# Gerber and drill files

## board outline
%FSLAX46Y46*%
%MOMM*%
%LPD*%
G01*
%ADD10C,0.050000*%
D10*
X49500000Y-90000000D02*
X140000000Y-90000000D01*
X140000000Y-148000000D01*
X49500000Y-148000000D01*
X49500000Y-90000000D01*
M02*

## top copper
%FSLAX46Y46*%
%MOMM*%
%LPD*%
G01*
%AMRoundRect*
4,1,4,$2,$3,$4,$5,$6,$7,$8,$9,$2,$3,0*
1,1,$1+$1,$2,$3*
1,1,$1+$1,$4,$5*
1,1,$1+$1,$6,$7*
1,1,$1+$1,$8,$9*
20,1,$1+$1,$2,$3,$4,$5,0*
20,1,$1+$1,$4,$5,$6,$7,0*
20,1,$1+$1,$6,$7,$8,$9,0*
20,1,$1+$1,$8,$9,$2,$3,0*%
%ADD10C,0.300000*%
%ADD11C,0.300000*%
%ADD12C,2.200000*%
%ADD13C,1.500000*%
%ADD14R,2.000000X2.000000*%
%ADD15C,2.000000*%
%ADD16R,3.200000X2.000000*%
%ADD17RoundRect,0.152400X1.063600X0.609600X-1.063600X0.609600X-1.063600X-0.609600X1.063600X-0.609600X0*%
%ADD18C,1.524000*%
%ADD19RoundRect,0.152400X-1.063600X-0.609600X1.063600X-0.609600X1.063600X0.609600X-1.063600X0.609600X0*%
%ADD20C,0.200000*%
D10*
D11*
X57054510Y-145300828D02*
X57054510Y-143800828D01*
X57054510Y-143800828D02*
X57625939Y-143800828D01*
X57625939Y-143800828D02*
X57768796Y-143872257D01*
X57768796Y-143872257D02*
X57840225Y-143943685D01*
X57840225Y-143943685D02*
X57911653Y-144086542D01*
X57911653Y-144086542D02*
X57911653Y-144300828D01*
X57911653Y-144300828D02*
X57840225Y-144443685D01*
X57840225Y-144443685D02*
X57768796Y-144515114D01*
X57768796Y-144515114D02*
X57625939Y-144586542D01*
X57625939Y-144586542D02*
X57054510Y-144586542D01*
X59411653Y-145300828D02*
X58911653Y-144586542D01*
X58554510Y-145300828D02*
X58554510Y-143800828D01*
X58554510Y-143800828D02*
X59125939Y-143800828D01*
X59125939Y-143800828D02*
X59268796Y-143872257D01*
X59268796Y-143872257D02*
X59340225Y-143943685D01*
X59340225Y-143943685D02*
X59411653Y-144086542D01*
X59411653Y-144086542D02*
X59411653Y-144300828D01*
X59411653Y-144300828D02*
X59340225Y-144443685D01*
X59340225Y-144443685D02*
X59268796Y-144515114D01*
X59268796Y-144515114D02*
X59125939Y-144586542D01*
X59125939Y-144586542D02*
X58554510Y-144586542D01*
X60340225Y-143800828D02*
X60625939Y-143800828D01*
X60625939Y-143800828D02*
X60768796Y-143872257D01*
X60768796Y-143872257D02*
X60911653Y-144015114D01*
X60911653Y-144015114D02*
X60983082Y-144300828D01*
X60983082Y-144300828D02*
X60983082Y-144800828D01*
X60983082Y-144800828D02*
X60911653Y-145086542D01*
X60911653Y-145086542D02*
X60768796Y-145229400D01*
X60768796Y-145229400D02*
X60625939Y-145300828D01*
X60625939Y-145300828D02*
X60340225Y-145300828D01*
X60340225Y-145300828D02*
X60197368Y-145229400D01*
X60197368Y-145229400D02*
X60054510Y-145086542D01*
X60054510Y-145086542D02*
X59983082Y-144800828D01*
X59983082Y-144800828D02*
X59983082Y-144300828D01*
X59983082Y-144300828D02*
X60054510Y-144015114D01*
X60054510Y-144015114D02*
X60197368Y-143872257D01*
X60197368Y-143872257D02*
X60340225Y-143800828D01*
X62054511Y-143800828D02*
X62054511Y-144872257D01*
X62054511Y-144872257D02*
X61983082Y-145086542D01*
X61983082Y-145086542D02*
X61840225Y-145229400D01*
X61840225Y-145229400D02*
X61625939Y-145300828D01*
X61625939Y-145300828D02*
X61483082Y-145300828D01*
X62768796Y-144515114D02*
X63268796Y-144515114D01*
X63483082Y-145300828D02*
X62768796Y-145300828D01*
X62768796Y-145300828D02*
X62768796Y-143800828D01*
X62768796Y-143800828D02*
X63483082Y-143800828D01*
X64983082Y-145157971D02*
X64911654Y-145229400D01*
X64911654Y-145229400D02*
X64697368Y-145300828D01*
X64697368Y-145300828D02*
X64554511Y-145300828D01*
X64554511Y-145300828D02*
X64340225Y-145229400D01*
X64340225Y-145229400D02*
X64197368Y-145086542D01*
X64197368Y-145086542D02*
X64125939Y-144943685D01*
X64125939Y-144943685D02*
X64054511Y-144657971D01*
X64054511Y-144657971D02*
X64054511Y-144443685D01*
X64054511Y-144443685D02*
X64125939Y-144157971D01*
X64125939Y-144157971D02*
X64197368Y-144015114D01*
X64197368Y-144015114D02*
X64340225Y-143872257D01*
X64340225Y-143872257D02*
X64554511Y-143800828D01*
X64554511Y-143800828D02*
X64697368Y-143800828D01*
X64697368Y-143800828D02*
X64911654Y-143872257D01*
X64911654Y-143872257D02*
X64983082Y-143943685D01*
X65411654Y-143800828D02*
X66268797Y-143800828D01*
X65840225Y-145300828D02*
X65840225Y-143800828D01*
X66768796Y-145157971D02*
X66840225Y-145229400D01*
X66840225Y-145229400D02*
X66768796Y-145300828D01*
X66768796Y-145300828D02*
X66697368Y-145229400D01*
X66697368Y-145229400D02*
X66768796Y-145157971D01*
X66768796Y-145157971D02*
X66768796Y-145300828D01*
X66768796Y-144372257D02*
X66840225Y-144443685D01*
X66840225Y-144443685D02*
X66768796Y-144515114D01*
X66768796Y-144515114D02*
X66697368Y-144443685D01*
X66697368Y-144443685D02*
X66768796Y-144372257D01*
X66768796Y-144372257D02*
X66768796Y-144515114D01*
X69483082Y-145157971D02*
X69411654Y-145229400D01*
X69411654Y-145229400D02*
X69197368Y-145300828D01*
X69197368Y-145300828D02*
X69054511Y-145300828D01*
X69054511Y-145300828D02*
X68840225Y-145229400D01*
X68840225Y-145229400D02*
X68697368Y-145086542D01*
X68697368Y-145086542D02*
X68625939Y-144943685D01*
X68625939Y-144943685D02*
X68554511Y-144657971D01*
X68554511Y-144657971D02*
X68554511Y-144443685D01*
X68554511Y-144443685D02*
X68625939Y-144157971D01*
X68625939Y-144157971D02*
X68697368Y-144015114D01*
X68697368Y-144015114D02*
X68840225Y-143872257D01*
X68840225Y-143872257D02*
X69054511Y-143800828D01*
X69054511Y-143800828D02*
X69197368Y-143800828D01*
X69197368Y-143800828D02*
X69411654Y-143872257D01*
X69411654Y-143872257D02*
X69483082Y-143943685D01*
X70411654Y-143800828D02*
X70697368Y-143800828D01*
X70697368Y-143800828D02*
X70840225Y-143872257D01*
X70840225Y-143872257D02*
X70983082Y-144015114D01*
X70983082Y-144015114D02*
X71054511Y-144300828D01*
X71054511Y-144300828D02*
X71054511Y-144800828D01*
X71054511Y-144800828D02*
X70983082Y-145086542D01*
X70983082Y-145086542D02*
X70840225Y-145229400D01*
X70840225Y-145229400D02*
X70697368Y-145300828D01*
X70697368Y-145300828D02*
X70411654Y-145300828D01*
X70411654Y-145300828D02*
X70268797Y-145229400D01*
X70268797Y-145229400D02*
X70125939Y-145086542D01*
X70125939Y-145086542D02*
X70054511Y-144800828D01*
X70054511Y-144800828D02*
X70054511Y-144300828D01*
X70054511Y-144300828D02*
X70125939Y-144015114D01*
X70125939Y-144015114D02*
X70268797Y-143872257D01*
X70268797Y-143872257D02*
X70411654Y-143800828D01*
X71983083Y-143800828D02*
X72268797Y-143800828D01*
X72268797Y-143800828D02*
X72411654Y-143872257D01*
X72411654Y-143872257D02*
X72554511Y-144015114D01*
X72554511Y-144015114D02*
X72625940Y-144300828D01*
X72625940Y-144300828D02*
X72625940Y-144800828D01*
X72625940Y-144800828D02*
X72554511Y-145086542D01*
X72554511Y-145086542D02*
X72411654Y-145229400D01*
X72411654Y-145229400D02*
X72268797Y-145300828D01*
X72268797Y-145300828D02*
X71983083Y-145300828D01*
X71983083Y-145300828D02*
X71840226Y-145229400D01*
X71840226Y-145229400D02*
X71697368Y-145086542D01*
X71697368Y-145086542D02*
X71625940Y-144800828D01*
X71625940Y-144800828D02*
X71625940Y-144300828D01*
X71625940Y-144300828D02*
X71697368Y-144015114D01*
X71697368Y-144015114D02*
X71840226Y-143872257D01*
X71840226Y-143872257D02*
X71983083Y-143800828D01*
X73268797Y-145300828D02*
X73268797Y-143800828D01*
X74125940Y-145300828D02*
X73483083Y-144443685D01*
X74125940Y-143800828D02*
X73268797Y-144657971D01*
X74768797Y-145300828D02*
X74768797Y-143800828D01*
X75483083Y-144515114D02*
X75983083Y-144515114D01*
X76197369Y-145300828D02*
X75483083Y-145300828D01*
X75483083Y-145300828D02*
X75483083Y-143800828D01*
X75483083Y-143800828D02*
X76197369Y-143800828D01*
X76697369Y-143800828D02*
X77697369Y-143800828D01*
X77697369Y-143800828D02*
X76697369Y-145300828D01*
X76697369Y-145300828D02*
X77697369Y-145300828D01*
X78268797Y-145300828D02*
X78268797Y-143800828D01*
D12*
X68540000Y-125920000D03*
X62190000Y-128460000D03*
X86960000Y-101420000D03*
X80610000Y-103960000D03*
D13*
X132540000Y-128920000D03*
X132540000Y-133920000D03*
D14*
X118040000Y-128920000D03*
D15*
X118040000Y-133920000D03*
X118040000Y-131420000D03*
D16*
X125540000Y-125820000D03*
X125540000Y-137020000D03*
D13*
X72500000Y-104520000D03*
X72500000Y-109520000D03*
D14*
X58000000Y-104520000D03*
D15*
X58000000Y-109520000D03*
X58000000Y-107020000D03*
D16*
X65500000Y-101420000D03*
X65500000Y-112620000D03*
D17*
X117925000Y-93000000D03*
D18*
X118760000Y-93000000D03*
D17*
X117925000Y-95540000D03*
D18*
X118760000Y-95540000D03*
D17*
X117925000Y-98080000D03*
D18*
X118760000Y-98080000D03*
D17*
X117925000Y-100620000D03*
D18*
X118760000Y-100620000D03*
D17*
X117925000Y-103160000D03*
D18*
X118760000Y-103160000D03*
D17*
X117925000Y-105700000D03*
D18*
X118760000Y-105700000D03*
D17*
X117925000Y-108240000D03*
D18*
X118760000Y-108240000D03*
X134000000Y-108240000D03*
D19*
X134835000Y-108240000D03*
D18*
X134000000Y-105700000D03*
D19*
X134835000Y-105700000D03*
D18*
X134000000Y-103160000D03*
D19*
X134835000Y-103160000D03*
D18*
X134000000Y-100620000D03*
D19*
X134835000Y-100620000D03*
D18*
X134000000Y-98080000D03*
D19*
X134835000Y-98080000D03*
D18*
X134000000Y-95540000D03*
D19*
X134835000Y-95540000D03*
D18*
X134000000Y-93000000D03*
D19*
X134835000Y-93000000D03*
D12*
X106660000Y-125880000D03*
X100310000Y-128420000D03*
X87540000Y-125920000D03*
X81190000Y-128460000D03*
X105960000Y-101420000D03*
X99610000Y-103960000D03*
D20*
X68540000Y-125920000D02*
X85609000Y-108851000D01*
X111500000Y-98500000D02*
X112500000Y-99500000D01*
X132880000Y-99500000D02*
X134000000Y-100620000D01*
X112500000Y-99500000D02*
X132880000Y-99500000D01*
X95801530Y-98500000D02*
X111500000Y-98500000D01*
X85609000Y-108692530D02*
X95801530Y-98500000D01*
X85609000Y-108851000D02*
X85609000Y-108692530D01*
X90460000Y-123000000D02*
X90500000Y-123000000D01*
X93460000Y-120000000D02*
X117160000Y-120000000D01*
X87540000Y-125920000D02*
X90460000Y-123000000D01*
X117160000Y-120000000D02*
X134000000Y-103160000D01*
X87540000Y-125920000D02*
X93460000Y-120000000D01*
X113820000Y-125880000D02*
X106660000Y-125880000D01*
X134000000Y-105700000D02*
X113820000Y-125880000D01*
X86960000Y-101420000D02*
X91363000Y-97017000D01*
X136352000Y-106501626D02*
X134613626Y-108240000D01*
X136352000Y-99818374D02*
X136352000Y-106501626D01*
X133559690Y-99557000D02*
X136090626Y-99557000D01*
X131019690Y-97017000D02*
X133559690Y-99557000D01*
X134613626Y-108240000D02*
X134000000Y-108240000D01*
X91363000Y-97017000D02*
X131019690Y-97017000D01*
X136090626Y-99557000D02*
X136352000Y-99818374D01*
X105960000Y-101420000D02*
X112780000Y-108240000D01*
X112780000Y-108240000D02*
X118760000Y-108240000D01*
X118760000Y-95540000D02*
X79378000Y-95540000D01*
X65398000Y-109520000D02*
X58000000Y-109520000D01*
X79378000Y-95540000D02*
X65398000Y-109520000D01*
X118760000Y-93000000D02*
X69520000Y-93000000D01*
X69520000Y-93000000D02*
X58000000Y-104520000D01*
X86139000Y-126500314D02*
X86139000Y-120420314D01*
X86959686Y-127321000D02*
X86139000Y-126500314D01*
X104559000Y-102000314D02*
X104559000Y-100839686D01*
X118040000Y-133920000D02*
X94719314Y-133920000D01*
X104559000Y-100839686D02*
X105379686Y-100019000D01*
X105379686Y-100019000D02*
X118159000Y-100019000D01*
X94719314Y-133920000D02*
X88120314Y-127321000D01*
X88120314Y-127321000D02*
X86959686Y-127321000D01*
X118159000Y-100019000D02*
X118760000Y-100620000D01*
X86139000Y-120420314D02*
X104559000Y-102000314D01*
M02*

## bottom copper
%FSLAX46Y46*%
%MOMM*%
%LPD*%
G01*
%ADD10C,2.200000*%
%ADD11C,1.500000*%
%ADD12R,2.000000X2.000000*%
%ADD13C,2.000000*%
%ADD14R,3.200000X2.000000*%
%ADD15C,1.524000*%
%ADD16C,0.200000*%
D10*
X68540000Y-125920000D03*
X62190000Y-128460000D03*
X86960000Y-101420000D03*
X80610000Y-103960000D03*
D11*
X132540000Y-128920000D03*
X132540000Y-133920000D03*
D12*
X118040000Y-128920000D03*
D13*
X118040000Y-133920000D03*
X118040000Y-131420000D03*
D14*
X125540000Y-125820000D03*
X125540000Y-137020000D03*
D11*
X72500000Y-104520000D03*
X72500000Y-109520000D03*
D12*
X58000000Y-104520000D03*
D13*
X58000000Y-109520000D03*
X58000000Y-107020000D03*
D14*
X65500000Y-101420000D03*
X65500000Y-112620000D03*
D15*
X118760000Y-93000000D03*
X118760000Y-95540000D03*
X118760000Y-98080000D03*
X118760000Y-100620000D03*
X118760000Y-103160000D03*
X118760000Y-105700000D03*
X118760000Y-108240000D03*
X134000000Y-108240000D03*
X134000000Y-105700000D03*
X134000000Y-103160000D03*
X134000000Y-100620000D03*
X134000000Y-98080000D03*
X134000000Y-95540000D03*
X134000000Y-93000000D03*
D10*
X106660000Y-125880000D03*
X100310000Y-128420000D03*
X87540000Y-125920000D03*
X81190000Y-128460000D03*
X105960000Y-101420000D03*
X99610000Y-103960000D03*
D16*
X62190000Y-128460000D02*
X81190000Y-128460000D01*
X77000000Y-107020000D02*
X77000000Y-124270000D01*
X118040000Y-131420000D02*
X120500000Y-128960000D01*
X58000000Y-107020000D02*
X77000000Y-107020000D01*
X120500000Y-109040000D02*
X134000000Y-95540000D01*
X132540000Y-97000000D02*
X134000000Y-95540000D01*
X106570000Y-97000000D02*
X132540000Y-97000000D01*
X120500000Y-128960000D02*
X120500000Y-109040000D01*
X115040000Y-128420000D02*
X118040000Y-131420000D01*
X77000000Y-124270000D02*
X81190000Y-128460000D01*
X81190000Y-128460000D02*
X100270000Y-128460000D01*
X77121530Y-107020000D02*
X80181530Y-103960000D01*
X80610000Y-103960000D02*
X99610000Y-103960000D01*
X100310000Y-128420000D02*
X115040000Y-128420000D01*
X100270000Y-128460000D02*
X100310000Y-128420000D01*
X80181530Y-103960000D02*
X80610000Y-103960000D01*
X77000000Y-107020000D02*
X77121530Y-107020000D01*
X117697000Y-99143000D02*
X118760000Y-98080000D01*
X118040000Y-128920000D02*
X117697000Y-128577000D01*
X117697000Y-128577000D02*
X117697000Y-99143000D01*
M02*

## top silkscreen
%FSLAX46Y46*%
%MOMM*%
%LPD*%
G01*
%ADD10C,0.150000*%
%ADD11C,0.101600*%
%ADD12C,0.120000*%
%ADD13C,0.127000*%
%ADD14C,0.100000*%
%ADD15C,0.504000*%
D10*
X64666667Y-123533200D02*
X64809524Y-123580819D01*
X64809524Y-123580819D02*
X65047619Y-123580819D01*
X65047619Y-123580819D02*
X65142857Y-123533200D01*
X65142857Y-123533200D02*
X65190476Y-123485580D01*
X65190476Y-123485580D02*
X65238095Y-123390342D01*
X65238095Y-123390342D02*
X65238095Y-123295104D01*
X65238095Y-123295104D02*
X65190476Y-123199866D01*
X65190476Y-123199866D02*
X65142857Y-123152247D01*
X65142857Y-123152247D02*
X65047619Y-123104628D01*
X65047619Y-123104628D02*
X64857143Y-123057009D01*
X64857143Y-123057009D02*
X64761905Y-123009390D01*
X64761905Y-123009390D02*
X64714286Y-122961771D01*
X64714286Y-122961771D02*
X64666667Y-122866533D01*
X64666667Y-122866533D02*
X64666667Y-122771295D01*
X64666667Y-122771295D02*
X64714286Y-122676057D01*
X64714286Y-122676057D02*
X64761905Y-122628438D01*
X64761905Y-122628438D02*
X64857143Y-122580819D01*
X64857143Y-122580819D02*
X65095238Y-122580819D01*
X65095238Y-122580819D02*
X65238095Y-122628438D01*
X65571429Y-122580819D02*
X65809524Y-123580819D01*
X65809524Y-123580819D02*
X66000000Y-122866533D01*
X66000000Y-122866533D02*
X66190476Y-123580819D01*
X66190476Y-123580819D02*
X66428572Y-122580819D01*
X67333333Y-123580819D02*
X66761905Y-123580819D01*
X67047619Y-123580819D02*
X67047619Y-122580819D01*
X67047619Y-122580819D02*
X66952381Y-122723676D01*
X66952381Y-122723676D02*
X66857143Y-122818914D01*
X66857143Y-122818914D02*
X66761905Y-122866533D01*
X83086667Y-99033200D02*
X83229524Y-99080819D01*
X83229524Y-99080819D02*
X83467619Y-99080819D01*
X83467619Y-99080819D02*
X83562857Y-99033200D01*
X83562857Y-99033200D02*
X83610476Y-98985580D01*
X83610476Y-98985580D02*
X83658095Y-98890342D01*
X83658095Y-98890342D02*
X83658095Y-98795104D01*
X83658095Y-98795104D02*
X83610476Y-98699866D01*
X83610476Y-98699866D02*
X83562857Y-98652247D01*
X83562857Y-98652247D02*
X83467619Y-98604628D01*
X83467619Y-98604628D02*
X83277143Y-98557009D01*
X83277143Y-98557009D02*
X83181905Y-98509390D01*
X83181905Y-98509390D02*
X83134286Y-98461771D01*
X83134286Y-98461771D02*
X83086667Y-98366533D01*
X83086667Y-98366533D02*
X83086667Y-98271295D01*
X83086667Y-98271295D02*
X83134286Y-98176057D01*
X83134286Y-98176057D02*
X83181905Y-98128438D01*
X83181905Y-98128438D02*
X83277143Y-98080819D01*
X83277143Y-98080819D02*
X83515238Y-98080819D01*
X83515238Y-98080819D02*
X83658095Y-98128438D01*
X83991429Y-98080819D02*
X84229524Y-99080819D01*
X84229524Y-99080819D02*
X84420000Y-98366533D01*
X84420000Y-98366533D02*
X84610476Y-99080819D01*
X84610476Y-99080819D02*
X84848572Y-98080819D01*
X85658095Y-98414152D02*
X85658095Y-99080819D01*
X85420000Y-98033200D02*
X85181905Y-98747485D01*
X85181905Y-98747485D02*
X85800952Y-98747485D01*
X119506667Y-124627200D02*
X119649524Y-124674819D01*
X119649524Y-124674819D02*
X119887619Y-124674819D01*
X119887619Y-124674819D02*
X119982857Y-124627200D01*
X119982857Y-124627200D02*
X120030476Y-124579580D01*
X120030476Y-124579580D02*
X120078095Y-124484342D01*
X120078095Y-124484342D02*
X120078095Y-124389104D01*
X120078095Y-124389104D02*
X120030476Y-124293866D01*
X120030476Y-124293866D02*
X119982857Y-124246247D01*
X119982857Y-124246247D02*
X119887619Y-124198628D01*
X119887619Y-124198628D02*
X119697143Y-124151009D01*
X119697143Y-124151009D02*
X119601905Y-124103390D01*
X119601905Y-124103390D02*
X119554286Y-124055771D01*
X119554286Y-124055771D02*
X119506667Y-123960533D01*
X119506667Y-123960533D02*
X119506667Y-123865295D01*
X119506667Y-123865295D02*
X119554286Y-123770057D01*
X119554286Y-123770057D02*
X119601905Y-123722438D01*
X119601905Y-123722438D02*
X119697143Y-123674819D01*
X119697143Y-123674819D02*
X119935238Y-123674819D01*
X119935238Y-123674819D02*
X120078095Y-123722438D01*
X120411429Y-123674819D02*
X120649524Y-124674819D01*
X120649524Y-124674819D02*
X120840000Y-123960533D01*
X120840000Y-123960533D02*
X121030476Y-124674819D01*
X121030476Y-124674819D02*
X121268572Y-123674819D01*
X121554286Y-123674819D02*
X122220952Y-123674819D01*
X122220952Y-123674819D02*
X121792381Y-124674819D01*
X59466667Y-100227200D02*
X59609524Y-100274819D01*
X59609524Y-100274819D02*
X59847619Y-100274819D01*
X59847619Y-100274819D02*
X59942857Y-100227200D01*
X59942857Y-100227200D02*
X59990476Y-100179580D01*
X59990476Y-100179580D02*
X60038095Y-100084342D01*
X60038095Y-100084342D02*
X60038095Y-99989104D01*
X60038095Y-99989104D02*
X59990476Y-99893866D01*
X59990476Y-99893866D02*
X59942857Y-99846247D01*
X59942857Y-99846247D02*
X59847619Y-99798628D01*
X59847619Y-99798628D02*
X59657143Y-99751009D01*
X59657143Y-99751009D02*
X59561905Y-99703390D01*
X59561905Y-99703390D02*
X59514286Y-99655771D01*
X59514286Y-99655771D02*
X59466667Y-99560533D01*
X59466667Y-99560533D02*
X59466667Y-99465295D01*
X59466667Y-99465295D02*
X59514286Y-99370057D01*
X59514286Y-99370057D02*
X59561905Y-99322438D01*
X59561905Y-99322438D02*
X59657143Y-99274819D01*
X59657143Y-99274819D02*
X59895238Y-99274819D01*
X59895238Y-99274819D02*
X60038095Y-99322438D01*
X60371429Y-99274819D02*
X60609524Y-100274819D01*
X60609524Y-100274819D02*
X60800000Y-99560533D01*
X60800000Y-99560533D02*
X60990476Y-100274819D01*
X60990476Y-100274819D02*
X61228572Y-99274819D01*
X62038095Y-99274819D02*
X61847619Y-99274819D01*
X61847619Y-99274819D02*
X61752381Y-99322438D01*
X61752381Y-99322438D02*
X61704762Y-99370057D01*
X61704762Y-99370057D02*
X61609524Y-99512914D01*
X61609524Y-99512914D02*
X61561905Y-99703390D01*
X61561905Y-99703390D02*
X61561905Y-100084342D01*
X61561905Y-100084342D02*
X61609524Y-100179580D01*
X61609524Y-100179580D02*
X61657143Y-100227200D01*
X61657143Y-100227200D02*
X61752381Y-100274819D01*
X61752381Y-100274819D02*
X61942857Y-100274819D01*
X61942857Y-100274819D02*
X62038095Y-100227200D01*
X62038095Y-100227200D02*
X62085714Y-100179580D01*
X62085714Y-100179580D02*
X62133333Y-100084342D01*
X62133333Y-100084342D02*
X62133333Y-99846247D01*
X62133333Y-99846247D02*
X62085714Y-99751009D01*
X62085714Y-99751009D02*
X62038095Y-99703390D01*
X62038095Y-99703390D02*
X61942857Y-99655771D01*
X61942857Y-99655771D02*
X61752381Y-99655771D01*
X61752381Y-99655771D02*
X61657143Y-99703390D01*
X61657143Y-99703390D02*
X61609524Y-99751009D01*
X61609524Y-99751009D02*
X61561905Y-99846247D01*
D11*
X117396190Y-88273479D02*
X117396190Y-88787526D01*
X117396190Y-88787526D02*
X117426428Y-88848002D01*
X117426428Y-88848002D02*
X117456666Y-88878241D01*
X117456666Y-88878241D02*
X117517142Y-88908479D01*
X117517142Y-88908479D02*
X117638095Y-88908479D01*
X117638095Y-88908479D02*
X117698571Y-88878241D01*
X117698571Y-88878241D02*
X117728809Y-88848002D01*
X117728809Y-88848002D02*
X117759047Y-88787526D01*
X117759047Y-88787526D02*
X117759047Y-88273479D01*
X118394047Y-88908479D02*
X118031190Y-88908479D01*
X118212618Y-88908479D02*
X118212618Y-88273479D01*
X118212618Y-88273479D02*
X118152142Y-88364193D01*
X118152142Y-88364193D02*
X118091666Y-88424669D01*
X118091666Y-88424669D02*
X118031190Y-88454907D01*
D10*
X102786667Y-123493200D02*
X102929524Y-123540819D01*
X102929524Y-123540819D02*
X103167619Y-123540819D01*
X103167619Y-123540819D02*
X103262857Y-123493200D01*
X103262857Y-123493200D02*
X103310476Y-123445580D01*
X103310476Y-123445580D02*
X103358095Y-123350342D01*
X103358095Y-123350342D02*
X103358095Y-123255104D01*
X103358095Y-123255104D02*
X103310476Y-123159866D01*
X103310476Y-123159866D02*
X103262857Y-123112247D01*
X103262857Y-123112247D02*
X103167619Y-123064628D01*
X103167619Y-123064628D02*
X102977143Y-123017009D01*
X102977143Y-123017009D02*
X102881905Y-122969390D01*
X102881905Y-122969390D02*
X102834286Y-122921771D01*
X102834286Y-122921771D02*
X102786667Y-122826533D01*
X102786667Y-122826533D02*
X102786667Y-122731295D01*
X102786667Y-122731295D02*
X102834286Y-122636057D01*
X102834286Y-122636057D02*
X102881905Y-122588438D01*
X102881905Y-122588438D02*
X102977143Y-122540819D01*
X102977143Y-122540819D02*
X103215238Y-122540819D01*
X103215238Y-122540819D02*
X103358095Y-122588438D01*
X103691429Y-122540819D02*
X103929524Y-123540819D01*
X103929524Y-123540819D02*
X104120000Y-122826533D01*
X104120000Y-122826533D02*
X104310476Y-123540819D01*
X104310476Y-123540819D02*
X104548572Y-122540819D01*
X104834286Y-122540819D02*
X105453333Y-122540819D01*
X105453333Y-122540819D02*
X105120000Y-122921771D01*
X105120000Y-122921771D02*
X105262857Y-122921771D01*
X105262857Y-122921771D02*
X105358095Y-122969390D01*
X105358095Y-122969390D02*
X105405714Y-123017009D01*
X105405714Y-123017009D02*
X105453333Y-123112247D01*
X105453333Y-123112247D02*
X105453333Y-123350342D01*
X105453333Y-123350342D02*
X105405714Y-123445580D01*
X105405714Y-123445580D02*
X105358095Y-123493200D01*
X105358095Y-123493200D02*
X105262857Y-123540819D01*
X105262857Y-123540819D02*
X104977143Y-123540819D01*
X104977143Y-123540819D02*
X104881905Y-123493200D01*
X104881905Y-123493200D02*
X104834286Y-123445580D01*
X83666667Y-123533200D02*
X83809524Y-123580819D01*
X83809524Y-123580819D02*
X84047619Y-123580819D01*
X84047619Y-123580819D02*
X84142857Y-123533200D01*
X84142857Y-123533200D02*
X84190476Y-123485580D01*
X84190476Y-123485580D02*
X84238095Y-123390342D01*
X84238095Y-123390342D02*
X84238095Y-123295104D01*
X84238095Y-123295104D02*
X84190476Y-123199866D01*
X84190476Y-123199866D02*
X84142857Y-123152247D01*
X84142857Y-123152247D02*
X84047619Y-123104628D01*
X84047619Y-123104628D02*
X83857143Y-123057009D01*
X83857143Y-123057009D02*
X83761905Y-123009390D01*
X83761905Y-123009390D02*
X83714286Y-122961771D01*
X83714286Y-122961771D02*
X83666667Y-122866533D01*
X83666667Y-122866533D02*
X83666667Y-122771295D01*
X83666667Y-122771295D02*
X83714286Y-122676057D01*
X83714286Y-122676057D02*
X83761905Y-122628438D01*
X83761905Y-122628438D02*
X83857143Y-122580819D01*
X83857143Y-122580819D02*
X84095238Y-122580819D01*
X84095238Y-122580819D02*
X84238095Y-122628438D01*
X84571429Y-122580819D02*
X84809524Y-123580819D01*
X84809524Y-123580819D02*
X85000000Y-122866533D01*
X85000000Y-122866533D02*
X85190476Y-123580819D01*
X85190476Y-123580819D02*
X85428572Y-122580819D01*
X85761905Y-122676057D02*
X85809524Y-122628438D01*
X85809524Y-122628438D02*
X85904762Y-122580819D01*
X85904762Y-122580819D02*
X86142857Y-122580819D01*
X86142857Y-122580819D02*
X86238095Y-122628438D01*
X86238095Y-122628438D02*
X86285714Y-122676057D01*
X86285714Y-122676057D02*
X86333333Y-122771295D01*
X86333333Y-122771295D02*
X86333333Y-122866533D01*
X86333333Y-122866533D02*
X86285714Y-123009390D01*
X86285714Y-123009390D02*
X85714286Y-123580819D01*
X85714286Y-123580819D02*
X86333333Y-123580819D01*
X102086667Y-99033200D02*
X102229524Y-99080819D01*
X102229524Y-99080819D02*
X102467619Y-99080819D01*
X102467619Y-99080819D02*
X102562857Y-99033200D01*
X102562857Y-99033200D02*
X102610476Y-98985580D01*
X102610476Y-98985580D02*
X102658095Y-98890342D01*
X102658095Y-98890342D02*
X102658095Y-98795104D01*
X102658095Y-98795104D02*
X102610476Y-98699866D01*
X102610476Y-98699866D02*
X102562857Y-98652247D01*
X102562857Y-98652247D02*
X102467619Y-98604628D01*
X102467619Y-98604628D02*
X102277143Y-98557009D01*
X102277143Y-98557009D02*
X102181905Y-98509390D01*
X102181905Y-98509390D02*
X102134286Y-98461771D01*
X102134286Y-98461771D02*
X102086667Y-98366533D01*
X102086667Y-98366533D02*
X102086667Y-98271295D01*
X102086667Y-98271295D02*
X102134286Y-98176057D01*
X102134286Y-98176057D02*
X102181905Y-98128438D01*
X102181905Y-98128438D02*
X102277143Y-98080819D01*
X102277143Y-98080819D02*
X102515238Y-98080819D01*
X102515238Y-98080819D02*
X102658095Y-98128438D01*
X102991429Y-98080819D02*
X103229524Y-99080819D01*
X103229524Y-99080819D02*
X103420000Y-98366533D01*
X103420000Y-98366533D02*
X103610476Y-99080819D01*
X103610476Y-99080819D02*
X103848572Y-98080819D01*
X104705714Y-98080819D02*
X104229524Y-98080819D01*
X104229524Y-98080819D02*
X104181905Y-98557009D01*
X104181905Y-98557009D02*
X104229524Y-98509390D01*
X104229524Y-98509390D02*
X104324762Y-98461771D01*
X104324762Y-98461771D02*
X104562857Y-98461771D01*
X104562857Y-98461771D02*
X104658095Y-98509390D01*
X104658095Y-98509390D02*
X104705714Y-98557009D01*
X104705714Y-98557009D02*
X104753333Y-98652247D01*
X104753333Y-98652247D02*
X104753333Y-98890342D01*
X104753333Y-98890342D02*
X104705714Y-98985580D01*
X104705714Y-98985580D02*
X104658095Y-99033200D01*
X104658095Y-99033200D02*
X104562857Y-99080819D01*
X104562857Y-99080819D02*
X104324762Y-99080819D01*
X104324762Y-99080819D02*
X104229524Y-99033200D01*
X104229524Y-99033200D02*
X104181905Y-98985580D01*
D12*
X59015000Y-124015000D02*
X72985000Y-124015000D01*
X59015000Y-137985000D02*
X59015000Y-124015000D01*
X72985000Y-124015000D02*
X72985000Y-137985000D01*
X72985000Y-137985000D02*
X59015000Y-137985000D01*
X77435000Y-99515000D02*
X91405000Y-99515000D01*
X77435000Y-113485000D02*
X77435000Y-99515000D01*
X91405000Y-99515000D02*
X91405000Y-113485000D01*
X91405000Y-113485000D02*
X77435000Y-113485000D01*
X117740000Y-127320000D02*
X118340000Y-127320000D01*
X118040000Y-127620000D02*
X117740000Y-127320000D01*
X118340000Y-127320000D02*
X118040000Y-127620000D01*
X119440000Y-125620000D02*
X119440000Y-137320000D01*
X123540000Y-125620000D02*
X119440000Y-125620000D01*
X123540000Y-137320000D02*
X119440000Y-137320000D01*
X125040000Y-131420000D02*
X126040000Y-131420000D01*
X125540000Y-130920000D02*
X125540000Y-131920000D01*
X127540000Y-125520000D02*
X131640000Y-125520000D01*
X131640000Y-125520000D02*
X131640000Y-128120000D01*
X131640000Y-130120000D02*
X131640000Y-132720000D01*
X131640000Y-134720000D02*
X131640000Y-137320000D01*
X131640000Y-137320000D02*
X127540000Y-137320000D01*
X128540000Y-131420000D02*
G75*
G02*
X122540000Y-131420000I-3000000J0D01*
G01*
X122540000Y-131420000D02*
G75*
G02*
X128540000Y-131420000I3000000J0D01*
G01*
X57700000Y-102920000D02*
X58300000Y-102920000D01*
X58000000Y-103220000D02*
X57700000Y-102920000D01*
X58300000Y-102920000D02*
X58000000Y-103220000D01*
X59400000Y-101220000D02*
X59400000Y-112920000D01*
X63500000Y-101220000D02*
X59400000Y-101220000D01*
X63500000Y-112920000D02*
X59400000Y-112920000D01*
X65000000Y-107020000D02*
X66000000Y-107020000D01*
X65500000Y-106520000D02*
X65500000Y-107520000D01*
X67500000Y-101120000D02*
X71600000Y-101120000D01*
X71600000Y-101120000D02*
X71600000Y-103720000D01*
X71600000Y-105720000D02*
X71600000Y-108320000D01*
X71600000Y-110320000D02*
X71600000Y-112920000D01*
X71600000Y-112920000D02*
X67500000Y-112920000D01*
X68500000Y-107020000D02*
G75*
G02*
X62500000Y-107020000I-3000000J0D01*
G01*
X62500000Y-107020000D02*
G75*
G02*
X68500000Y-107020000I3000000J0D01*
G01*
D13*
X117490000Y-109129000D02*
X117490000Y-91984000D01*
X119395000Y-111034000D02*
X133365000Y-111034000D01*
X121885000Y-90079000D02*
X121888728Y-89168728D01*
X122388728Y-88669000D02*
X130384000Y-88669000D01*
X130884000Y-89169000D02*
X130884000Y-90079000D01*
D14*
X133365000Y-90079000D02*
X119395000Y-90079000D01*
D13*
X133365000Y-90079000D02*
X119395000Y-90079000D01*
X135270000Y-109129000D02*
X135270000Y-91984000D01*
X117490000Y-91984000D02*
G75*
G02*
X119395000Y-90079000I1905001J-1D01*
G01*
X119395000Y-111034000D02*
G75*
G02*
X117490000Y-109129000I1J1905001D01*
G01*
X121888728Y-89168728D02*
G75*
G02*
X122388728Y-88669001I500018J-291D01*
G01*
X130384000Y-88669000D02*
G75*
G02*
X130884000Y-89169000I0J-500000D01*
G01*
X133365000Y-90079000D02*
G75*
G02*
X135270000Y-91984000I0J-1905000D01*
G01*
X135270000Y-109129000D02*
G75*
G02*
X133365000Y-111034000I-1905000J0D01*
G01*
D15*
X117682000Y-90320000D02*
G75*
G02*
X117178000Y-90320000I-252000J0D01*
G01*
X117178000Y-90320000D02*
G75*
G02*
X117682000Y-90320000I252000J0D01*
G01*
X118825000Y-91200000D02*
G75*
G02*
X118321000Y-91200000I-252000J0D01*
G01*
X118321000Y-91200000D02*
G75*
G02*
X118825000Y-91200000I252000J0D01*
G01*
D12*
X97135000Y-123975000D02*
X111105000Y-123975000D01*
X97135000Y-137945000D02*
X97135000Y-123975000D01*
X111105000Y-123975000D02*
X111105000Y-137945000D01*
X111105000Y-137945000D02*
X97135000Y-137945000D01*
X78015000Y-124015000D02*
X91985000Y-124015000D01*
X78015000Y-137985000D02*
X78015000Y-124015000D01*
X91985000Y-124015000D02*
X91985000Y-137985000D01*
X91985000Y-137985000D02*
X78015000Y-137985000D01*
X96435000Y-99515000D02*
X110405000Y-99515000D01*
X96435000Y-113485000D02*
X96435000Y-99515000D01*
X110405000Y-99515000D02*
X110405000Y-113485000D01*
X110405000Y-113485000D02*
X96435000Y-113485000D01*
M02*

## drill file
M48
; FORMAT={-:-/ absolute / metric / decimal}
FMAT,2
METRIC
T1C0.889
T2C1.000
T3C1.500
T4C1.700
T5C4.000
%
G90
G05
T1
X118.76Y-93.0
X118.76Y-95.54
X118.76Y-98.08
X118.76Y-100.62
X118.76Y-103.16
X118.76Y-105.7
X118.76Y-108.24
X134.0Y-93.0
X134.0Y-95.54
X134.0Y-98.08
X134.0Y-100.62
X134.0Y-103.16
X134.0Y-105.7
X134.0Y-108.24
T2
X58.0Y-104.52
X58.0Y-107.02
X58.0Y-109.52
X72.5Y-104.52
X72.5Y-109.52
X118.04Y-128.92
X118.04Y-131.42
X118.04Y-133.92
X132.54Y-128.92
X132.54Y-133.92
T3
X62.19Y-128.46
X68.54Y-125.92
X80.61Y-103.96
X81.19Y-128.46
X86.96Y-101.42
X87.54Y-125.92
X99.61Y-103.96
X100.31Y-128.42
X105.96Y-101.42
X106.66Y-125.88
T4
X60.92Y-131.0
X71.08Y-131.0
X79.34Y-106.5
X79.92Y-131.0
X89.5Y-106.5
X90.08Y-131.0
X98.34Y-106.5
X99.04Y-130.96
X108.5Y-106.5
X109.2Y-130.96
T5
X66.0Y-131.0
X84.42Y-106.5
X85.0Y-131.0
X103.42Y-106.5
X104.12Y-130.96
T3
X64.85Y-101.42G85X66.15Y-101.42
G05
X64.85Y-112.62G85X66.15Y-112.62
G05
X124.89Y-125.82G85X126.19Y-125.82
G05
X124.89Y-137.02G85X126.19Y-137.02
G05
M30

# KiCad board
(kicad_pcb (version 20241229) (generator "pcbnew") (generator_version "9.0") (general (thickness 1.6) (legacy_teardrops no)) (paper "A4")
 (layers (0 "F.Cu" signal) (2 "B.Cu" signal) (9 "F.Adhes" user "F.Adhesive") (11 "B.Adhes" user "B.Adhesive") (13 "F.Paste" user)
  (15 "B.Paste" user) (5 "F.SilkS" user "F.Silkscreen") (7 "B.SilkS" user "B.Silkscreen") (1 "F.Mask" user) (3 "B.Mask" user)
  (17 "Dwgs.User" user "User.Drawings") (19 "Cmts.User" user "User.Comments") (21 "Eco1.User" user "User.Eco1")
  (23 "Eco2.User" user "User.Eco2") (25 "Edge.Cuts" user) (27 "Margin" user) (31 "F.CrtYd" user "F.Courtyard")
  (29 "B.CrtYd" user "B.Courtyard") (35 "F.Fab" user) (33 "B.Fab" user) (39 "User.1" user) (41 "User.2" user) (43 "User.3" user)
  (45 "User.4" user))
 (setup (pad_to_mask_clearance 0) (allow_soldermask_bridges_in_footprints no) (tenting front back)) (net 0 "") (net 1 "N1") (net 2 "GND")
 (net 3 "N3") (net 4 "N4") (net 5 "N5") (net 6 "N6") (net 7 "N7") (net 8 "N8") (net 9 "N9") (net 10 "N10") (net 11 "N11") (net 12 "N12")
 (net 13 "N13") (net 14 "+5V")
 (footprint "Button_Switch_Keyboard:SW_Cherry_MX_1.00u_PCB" (layer "F.Cu") (at 68.54 125.92)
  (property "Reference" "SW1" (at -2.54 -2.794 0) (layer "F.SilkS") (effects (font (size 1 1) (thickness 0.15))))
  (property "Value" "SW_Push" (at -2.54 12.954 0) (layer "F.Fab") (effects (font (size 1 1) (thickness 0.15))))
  (fp_line (start -9.525 -1.905) (end 4.445 -1.905) (stroke (width 0.12) (type solid)) (layer "F.SilkS"))
  (fp_line (start -9.525 12.065) (end -9.525 -1.905) (stroke (width 0.12) (type solid)) (layer "F.SilkS"))
  (fp_line (start 4.445 -1.905) (end 4.445 12.065) (stroke (width 0.12) (type solid)) (layer "F.SilkS"))
  (fp_line (start 4.445 12.065) (end -9.525 12.065) (stroke (width 0.12) (type solid)) (layer "F.SilkS"))
  (pad "" np_thru_hole circle (at -7.62 5.08) (size 1.7 1.7) (drill 1.7) (layers "*.Cu" "*.Mask"))
  (pad "" np_thru_hole circle (at -2.54 5.08) (size 4 4) (drill 4) (layers "*.Cu" "*.Mask"))
  (pad "" np_thru_hole circle (at 2.54 5.08) (size 1.7 1.7) (drill 1.7) (layers "*.Cu" "*.Mask"))
  (pad "1" thru_hole circle (at 0 0) (size 2.2 2.2) (drill 1.5) (layers "*.Cu" "*.Mask") (remove_unused_layers no) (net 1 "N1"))
  (pad "2" thru_hole circle (at -6.35 2.54) (size 2.2 2.2) (drill 1.5) (layers "*.Cu" "*.Mask") (remove_unused_layers no) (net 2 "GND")))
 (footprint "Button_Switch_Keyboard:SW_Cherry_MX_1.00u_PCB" (layer "F.Cu") (at 86.96 101.42)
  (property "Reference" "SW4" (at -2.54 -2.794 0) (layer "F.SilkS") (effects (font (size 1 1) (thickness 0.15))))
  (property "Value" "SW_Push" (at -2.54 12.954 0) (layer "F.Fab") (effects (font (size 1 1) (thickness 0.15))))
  (fp_line (start -9.525 -1.905) (end 4.445 -1.905) (stroke (width 0.12) (type solid)) (layer "F.SilkS"))
  (fp_line (start -9.525 12.065) (end -9.525 -1.905) (stroke (width 0.12) (type solid)) (layer "F.SilkS"))
  (fp_line (start 4.445 -1.905) (end 4.445 12.065) (stroke (width 0.12) (type solid)) (layer "F.SilkS"))
  (fp_line (start 4.445 12.065) (end -9.525 12.065) (stroke (width 0.12) (type solid)) (layer "F.SilkS"))
  (pad "" np_thru_hole circle (at -7.62 5.08) (size 1.7 1.7) (drill 1.7) (layers "*.Cu" "*.Mask"))
  (pad "" np_thru_hole circle (at -2.54 5.08) (size 4 4) (drill 4) (layers "*.Cu" "*.Mask"))
  (pad "" np_thru_hole circle (at 2.54 5.08) (size 1.7 1.7) (drill 1.7) (layers "*.Cu" "*.Mask"))
  (pad "1" thru_hole circle (at 0 0) (size 2.2 2.2) (drill 1.5) (layers "*.Cu" "*.Mask") (remove_unused_layers no) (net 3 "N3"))
  (pad "2" thru_hole circle (at -6.35 2.54) (size 2.2 2.2) (drill 1.5) (layers "*.Cu" "*.Mask") (remove_unused_layers no) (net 2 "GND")))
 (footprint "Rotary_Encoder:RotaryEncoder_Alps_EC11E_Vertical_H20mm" (layer "F.Cu") (at 118.04 128.92)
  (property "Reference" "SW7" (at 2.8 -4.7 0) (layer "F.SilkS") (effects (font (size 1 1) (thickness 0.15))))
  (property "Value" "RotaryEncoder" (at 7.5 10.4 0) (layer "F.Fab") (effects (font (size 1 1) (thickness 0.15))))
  (fp_line (start -0.3 -1.6) (end 0.3 -1.6) (stroke (width 0.12) (type solid)) (layer "F.SilkS"))
  (fp_line (start 0 -1.3) (end -0.3 -1.6) (stroke (width 0.12) (type solid)) (layer "F.SilkS"))
  (fp_line (start 0.3 -1.6) (end 0 -1.3) (stroke (width 0.12) (type solid)) (layer "F.SilkS"))
  (fp_line (start 1.4 -3.3) (end 1.4 8.4) (stroke (width 0.12) (type solid)) (layer "F.SilkS"))
  (fp_line (start 5.5 -3.3) (end 1.4 -3.3) (stroke (width 0.12) (type solid)) (layer "F.SilkS"))
  (fp_line (start 5.5 8.4) (end 1.4 8.4) (stroke (width 0.12) (type solid)) (layer "F.SilkS"))
  (fp_line (start 7 2.5) (end 8 2.5) (stroke (width 0.12) (type solid)) (layer "F.SilkS"))
  (fp_line (start 7.5 2) (end 7.5 3) (stroke (width 0.12) (type solid)) (layer "F.SilkS"))
  (fp_line (start 9.5 -3.4) (end 13.6 -3.4) (stroke (width 0.12) (type solid)) (layer "F.SilkS"))
  (fp_line (start 13.6 -3.4) (end 13.6 -0.8) (stroke (width 0.12) (type solid)) (layer "F.SilkS"))
  (fp_line (start 13.6 1.2) (end 13.6 3.8) (stroke (width 0.12) (type solid)) (layer "F.SilkS"))
  (fp_line (start 13.6 5.8) (end 13.6 8.4) (stroke (width 0.12) (type solid)) (layer "F.SilkS"))
  (fp_line (start 13.6 8.4) (end 9.5 8.4) (stroke (width 0.12) (type solid)) (layer "F.SilkS"))
  (fp_circle (center 7.5 2.5) (end 10.5 2.5) (stroke (width 0.12) (type solid)) (fill no) (layer "F.SilkS"))
  (pad "" thru_hole circle (at 14.5 0) (size 1.5 1.5) (drill 1) (layers "*.Cu" "*.Mask") (remove_unused_layers no))
  (pad "" thru_hole circle (at 14.5 5) (size 1.5 1.5) (drill 1) (layers "*.Cu" "*.Mask") (remove_unused_layers no))
  (pad "A" thru_hole rect (at 0 0) (size 2 2) (drill 1) (layers "*.Cu" "*.Mask") (remove_unused_layers no) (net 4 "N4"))
  (pad "B" thru_hole circle (at 0 5) (size 2 2) (drill 1) (layers "*.Cu" "*.Mask") (remove_unused_layers no) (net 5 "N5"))
  (pad "C" thru_hole circle (at 0 2.5) (size 2 2) (drill 1) (layers "*.Cu" "*.Mask") (remove_unused_layers no) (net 2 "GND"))
  (pad "MP" thru_hole rect (at 7.5 -3.1) (size 3.2 2) (drill oval 2.8 1.5) (layers "*.Cu" "*.Mask") (remove_unused_layers no))
  (pad "MP" thru_hole rect (at 7.5 8.1) (size 3.2 2) (drill oval 2.8 1.5) (layers "*.Cu" "*.Mask") (remove_unused_layers no)))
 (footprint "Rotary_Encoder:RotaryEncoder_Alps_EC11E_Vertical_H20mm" (layer "F.Cu") (at 58 104.52)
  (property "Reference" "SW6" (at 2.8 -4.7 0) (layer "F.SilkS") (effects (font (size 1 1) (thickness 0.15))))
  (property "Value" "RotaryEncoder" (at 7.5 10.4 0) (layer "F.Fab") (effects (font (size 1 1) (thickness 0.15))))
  (fp_line (start -0.3 -1.6) (end 0.3 -1.6) (stroke (width 0.12) (type solid)) (layer "F.SilkS"))
  (fp_line (start 0 -1.3) (end -0.3 -1.6) (stroke (width 0.12) (type solid)) (layer "F.SilkS"))
  (fp_line (start 0.3 -1.6) (end 0 -1.3) (stroke (width 0.12) (type solid)) (layer "F.SilkS"))
  (fp_line (start 1.4 -3.3) (end 1.4 8.4) (stroke (width 0.12) (type solid)) (layer "F.SilkS"))
  (fp_line (start 5.5 -3.3) (end 1.4 -3.3) (stroke (width 0.12) (type solid)) (layer "F.SilkS"))
  (fp_line (start 5.5 8.4) (end 1.4 8.4) (stroke (width 0.12) (type solid)) (layer "F.SilkS"))
  (fp_line (start 7 2.5) (end 8 2.5) (stroke (width 0.12) (type solid)) (layer "F.SilkS"))
  (fp_line (start 7.5 2) (end 7.5 3) (stroke (width 0.12) (type solid)) (layer "F.SilkS"))
  (fp_line (start 9.5 -3.4) (end 13.6 -3.4) (stroke (width 0.12) (type solid)) (layer "F.SilkS"))
  (fp_line (start 13.6 -3.4) (end 13.6 -0.8) (stroke (width 0.12) (type solid)) (layer "F.SilkS"))
  (fp_line (start 13.6 1.2) (end 13.6 3.8) (stroke (width 0.12) (type solid)) (layer "F.SilkS"))
  (fp_line (start 13.6 5.8) (end 13.6 8.4) (stroke (width 0.12) (type solid)) (layer "F.SilkS"))
  (fp_line (start 13.6 8.4) (end 9.5 8.4) (stroke (width 0.12) (type solid)) (layer "F.SilkS"))
  (fp_circle (center 7.5 2.5) (end 10.5 2.5) (stroke (width 0.12) (type solid)) (fill no) (layer "F.SilkS"))
  (pad "" thru_hole circle (at 14.5 0) (size 1.5 1.5) (drill 1) (layers "*.Cu" "*.Mask") (remove_unused_layers no))
  (pad "" thru_hole circle (at 14.5 5) (size 1.5 1.5) (drill 1) (layers "*.Cu" "*.Mask") (remove_unused_layers no))
  (pad "A" thru_hole rect (at 0 0) (size 2 2) (drill 1) (layers "*.Cu" "*.Mask") (remove_unused_layers no) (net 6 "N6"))
  (pad "B" thru_hole circle (at 0 5) (size 2 2) (drill 1) (layers "*.Cu" "*.Mask") (remove_unused_layers no) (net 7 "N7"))
  (pad "C" thru_hole circle (at 0 2.5) (size 2 2) (drill 1) (layers "*.Cu" "*.Mask") (remove_unused_layers no) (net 2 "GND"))
  (pad "MP" thru_hole rect (at 7.5 -3.1) (size 3.2 2) (drill oval 2.8 1.5) (layers "*.Cu" "*.Mask") (remove_unused_layers no))
  (pad "MP" thru_hole rect (at 7.5 8.1) (size 3.2 2) (drill oval 2.8 1.5) (layers "*.Cu" "*.Mask") (remove_unused_layers no)))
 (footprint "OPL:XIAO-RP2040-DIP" (layer "F.Cu") (at 126.38 100.62)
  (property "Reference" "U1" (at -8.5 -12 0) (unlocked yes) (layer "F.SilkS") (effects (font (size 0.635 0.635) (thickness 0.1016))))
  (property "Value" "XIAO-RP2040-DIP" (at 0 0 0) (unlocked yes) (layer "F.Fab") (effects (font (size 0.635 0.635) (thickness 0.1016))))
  (fp_line (start -8.89 8.509) (end -8.89 -8.636) (stroke (width 0.127) (type solid)) (layer "F.SilkS"))
  (fp_line (start -6.985 10.414) (end 6.985 10.414) (stroke (width 0.127) (type solid)) (layer "F.SilkS"))
  (fp_line (start -4.495 -10.541) (end -4.491272 -11.451272) (stroke (width 0.127) (type solid)) (layer "F.SilkS"))
  (fp_line (start -3.991272 -11.951) (end 4.004 -11.951) (stroke (width 0.127) (type solid)) (layer "F.SilkS"))
  (fp_line (start 4.504 -11.451) (end 4.504 -10.541) (stroke (width 0.127) (type solid)) (layer "F.SilkS"))
  (fp_line (start 6.985 -10.541) (end -6.985 -10.541) (stroke (width 0.1) (type solid)) (layer "F.SilkS"))
  (fp_line (start 6.985 -10.541) (end -6.985 -10.541) (stroke (width 0.127) (type solid)) (layer "F.SilkS"))
  (fp_line (start 8.89 8.509) (end 8.89 -8.636) (stroke (width 0.127) (type solid)) (layer "F.SilkS"))
  (fp_arc (start -8.89 -8.636) (mid -8.332038 -9.983038) (end -6.985 -10.541) (stroke (width 0.127) (type solid)) (layer "F.SilkS"))
  (fp_arc (start -6.985 10.414) (mid -8.332038 9.856038) (end -8.89 8.509) (stroke (width 0.127) (type solid)) (layer "F.SilkS"))
  (fp_arc (start -4.491272 -11.451272) (mid -4.344728 -11.80464) (end -3.991272 -11.951) (stroke (width 0.127) (type default))
   (layer "F.SilkS"))
  (fp_arc (start 4.004 -11.951) (mid 4.357553 -11.804553) (end 4.504 -11.451) (stroke (width 0.127) (type default)) (layer "F.SilkS"))
  (fp_arc (start 6.985 -10.541) (mid 8.332038 -9.983038) (end 8.89 -8.636) (stroke (width 0.127) (type solid)) (layer "F.SilkS"))
  (fp_arc (start 8.89 8.509) (mid 8.332038 9.856038) (end 6.985 10.414) (stroke (width 0.127) (type solid)) (layer "F.SilkS"))
  (fp_circle (center -8.95 -10.3) (end -8.95 -10.554) (stroke (width 0.5) (type solid)) (fill yes) (layer "F.SilkS"))
  (fp_circle (center -7.807 -9.42) (end -7.807 -9.674) (stroke (width 0.5) (type solid)) (fill yes) (layer "F.SilkS"))
  (pad "1" smd roundrect (at -8.455 -7.62 180) (size 2.432 1.524) (layers "F.Cu" "F.Mask") (roundrect_rratio 0.1) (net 6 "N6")
   (thermal_bridge_angle 45))
  (pad "1" thru_hole circle (at -7.62 -7.62 180) (size 1.524 1.524) (drill 0.889) (layers "*.Cu" "*.Mask") (remove_unused_layers no)
   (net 6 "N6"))
  (pad "2" smd roundrect (at -8.455 -5.08 180) (size 2.432 1.524) (layers "F.Cu" "F.Mask") (roundrect_rratio 0.1) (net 7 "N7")
   (thermal_bridge_angle 45))
  (pad "2" thru_hole circle (at -7.62 -5.08 180) (size 1.524 1.524) (drill 0.889) (layers "*.Cu" "*.Mask") (remove_unused_layers no)
   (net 7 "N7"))
  (pad "3" smd roundrect (at -8.455 -2.54 180) (size 2.432 1.524) (layers "F.Cu" "F.Mask") (roundrect_rratio 0.1) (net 4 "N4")
   (thermal_bridge_angle 45))
  (pad "3" thru_hole circle (at -7.62 -2.54 180) (size 1.524 1.524) (drill 0.889) (layers "*.Cu" "*.Mask") (remove_unused_layers no)
   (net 4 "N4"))
  (pad "4" smd roundrect (at -8.455 0 180) (size 2.432 1.524) (layers "F.Cu" "F.Mask") (roundrect_rratio 0.1) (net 5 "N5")
   (thermal_bridge_angle 45))
  (pad "4" thru_hole circle (at -7.62 0 180) (size 1.524 1.524) (drill 0.889) (layers "*.Cu" "*.Mask") (remove_unused_layers no)
   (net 5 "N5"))
  (pad "5" smd roundrect (at -8.455 2.54 180) (size 2.432 1.524) (layers "F.Cu" "F.Mask") (roundrect_rratio 0.1) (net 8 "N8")
   (thermal_bridge_angle 45))
  (pad "5" thru_hole circle (at -7.62 2.54 180) (size 1.524 1.524) (drill 0.889) (layers "*.Cu" "*.Mask") (remove_unused_layers no)
   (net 8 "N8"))
  (pad "6" smd roundrect (at -8.455 5.08 180) (size 2.432 1.524) (layers "F.Cu" "F.Mask") (roundrect_rratio 0.1) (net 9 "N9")
   (thermal_bridge_angle 45))
  (pad "6" thru_hole circle (at -7.62 5.08 180) (size 1.524 1.524) (drill 0.889) (layers "*.Cu" "*.Mask") (remove_unused_layers no)
   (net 9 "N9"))
  (pad "7" smd roundrect (at -8.455 7.62 180) (size 2.432 1.524) (layers "F.Cu" "F.Mask") (roundrect_rratio 0.1) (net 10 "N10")
   (thermal_bridge_angle 45))
  (pad "7" thru_hole circle (at -7.62 7.62 180) (size 1.524 1.524) (drill 0.889) (layers "*.Cu" "*.Mask") (remove_unused_layers no)
   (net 10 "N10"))
  (pad "8" thru_hole circle (at 7.62 7.62) (size 1.524 1.524) (drill 0.889) (layers "*.Cu" "*.Mask") (remove_unused_layers no) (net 3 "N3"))
  (pad "8" smd roundrect (at 8.455 7.62) (size 2.432 1.524) (layers "F.Cu" "F.Mask") (roundrect_rratio 0.1) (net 3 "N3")
   (thermal_bridge_angle 45))
  (pad "9" thru_hole circle (at 7.62 5.08) (size 1.524 1.524) (drill 0.889) (layers "*.Cu" "*.Mask") (remove_unused_layers no)
   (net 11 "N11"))
  (pad "9" smd roundrect (at 8.455 5.08) (size 2.432 1.524) (layers "F.Cu" "F.Mask") (roundrect_rratio 0.1) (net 11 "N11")
   (thermal_bridge_angle 45))
  (pad "10" thru_hole circle (at 7.62 2.54) (size 1.524 1.524) (drill 0.889) (layers "*.Cu" "*.Mask") (remove_unused_layers no)
   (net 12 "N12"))
  (pad "10" smd roundrect (at 8.455 2.54) (size 2.432 1.524) (layers "F.Cu" "F.Mask") (roundrect_rratio 0.1) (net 12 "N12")
   (thermal_bridge_angle 45))
  (pad "11" thru_hole circle (at 7.62 0) (size 1.524 1.524) (drill 0.889) (layers "*.Cu" "*.Mask") (remove_unused_layers no) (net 1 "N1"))
  (pad "11" smd roundrect (at 8.455 0) (size 2.432 1.524) (layers "F.Cu" "F.Mask") (roundrect_rratio 0.1) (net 1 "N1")
   (thermal_bridge_angle 45))
  (pad "12" thru_hole circle (at 7.62 -2.54) (size 1.524 1.524) (drill 0.889) (layers "*.Cu" "*.Mask") (remove_unused_layers no)
   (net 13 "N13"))
  (pad "12" smd roundrect (at 8.455 -2.54) (size 2.432 1.524) (layers "F.Cu" "F.Mask") (roundrect_rratio 0.1) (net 13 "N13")
   (thermal_bridge_angle 45))
  (pad "13" thru_hole circle (at 7.62 -5.08) (size 1.524 1.524) (drill 0.889) (layers "*.Cu" "*.Mask") (remove_unused_layers no)
   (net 2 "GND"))
  (pad "13" smd roundrect (at 8.455 -5.08) (size 2.432 1.524) (layers "F.Cu" "F.Mask") (roundrect_rratio 0.1) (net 2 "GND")
   (thermal_bridge_angle 45))
  (pad "14" thru_hole circle (at 7.62 -7.62) (size 1.524 1.524) (drill 0.889) (layers "*.Cu" "*.Mask") (remove_unused_layers no)
   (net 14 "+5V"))
  (pad "14" smd roundrect (at 8.455 -7.62) (size 2.432 1.524) (layers "F.Cu" "F.Mask") (roundrect_rratio 0.1) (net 14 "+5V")
   (thermal_bridge_angle 45)))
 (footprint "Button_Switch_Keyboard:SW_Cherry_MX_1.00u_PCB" (layer "F.Cu") (at 106.66 125.88)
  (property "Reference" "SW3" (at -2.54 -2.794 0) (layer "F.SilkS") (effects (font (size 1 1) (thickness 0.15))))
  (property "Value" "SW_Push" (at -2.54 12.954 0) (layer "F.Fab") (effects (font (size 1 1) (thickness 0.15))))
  (fp_line (start -9.525 -1.905) (end 4.445 -1.905) (stroke (width 0.12) (type solid)) (layer "F.SilkS"))
  (fp_line (start -9.525 12.065) (end -9.525 -1.905) (stroke (width 0.12) (type solid)) (layer "F.SilkS"))
  (fp_line (start 4.445 -1.905) (end 4.445 12.065) (stroke (width 0.12) (type solid)) (layer "F.SilkS"))
  (fp_line (start 4.445 12.065) (end -9.525 12.065) (stroke (width 0.12) (type solid)) (layer "F.SilkS"))
  (pad "" np_thru_hole circle (at -7.62 5.08) (size 1.7 1.7) (drill 1.7) (layers "*.Cu" "*.Mask"))
  (pad "" np_thru_hole circle (at -2.54 5.08) (size 4 4) (drill 4) (layers "*.Cu" "*.Mask"))
  (pad "" np_thru_hole circle (at 2.54 5.08) (size 1.7 1.7) (drill 1.7) (layers "*.Cu" "*.Mask"))
  (pad "1" thru_hole circle (at 0 0) (size 2.2 2.2) (drill 1.5) (layers "*.Cu" "*.Mask") (remove_unused_layers no) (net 11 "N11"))
  (pad "2" thru_hole circle (at -6.35 2.54) (size 2.2 2.2) (drill 1.5) (layers "*.Cu" "*.Mask") (remove_unused_layers no) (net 2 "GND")))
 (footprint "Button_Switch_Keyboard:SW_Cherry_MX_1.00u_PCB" (layer "F.Cu") (at 87.54 125.92)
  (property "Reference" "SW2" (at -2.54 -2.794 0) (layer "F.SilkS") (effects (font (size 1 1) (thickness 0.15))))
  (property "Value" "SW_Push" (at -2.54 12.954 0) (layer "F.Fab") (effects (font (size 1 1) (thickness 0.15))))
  (fp_line (start -9.525 -1.905) (end 4.445 -1.905) (stroke (width 0.12) (type solid)) (layer "F.SilkS"))
  (fp_line (start -9.525 12.065) (end -9.525 -1.905) (stroke (width 0.12) (type solid)) (layer "F.SilkS"))
  (fp_line (start 4.445 -1.905) (end 4.445 12.065) (stroke (width 0.12) (type solid)) (layer "F.SilkS"))
  (fp_line (start 4.445 12.065) (end -9.525 12.065) (stroke (width 0.12) (type solid)) (layer "F.SilkS"))
  (pad "" np_thru_hole circle (at -7.62 5.08) (size 1.7 1.7) (drill 1.7) (layers "*.Cu" "*.Mask"))
  (pad "" np_thru_hole circle (at -2.54 5.08) (size 4 4) (drill 4) (layers "*.Cu" "*.Mask"))
  (pad "" np_thru_hole circle (at 2.54 5.08) (size 1.7 1.7) (drill 1.7) (layers "*.Cu" "*.Mask"))
  (pad "1" thru_hole circle (at 0 0) (size 2.2 2.2) (drill 1.5) (layers "*.Cu" "*.Mask") (remove_unused_layers no) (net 12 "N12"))
  (pad "2" thru_hole circle (at -6.35 2.54) (size 2.2 2.2) (drill 1.5) (layers "*.Cu" "*.Mask") (remove_unused_layers no) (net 2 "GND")))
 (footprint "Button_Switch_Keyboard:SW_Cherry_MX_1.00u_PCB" (layer "F.Cu") (at 105.96 101.42)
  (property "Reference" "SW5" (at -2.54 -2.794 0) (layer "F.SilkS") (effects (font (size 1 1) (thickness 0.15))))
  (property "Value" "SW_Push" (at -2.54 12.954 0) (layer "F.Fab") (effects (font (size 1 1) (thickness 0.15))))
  (fp_line (start -9.525 -1.905) (end 4.445 -1.905) (stroke (width 0.12) (type solid)) (layer "F.SilkS"))
  (fp_line (start -9.525 12.065) (end -9.525 -1.905) (stroke (width 0.12) (type solid)) (layer "F.SilkS"))
  (fp_line (start 4.445 -1.905) (end 4.445 12.065) (stroke (width 0.12) (type solid)) (layer "F.SilkS"))
  (fp_line (start 4.445 12.065) (end -9.525 12.065) (stroke (width 0.12) (type solid)) (layer "F.SilkS"))
  (pad "" np_thru_hole circle (at -7.62 5.08) (size 1.7 1.7) (drill 1.7) (layers "*.Cu" "*.Mask"))
  (pad "" np_thru_hole circle (at -2.54 5.08) (size 4 4) (drill 4) (layers "*.Cu" "*.Mask"))
  (pad "" np_thru_hole circle (at 2.54 5.08) (size 1.7 1.7) (drill 1.7) (layers "*.Cu" "*.Mask"))
  (pad "1" thru_hole circle (at 0 0) (size 2.2 2.2) (drill 1.5) (layers "*.Cu" "*.Mask") (remove_unused_layers no) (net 10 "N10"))
  (pad "2" thru_hole circle (at -6.35 2.54) (size 2.2 2.2) (drill 1.5) (layers "*.Cu" "*.Mask") (remove_unused_layers no) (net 2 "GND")))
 (gr_rect (start 49.5 90) (end 140 148) (stroke (width 0.05) (type default)) (fill no) (layer "Edge.Cuts"))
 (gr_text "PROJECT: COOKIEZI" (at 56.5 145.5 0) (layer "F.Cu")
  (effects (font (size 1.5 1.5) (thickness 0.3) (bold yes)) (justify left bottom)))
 (segment (start 62.19 128.46) (end 81.19 128.46) (width 0.2) (layer "B.Cu") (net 2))
 (segment (start 77 107.02) (end 77 124.27) (width 0.2) (layer "B.Cu") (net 2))
 (segment (start 118.04 131.42) (end 120.5 128.96) (width 0.2) (layer "B.Cu") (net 2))
 (segment (start 58 107.02) (end 77 107.02) (width 0.2) (layer "B.Cu") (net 2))
 (segment (start 120.5 109.04) (end 134 95.54) (width 0.2) (layer "B.Cu") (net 2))
 (segment (start 132.54 97) (end 134 95.54) (width 0.2) (layer "B.Cu") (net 2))
 (segment (start 106.57 97) (end 132.54 97) (width 0.2) (layer "B.Cu") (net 2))
 (segment (start 120.5 128.96) (end 120.5 109.04) (width 0.2) (layer "B.Cu") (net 2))
 (segment (start 115.04 128.42) (end 118.04 131.42) (width 0.2) (layer "B.Cu") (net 2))
 (segment (start 77 124.27) (end 81.19 128.46) (width 0.2) (layer "B.Cu") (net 2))
 (segment (start 81.19 128.46) (end 100.27 128.46) (width 0.2) (layer "B.Cu") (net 2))
 (segment (start 77.12153 107.02) (end 80.18153 103.96) (width 0.2) (layer "B.Cu") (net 2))
 (segment (start 80.61 103.96) (end 99.61 103.96) (width 0.2) (layer "B.Cu") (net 2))
 (segment (start 100.31 128.42) (end 115.04 128.42) (width 0.2) (layer "B.Cu") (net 2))
 (segment (start 100.27 128.46) (end 100.31 128.42) (width 0.2) (layer "B.Cu") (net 2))
 (segment (start 80.18153 103.96) (end 80.61 103.96) (width 0.2) (layer "B.Cu") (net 2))
 (segment (start 77 107.02) (end 77.12153 107.02) (width 0.2) (layer "B.Cu") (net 2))
 (segment (start 68.54 125.92) (end 85.609 108.851) (width 0.2) (layer "F.Cu") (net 1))
 (segment (start 111.5 98.5) (end 112.5 99.5) (width 0.2) (layer "F.Cu") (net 1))
 (segment (start 132.88 99.5) (end 134 100.62) (width 0.2) (layer "F.Cu") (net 1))
 (segment (start 112.5 99.5) (end 132.88 99.5) (width 0.2) (layer "F.Cu") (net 1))
 (segment (start 95.80153 98.5) (end 111.5 98.5) (width 0.2) (layer "F.Cu") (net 1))
 (segment (start 85.609 108.69253) (end 95.80153 98.5) (width 0.2) (layer "F.Cu") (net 1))
 (segment (start 85.609 108.851) (end 85.609 108.69253) (width 0.2) (layer "F.Cu") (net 1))
 (segment (start 90.46 123) (end 90.5 123) (width 0.2) (layer "F.Cu") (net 12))
 (segment (start 93.46 120) (end 117.16 120) (width 0.2) (layer "F.Cu") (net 12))
 (segment (start 87.54 125.92) (end 90.46 123) (width 0.2) (layer "F.Cu") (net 12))
 (segment (start 117.16 120) (end 134 103.16) (width 0.2) (layer "F.Cu") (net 12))
 (segment (start 87.54 125.92) (end 93.46 120) (width 0.2) (layer "F.Cu") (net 12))
 (segment (start 113.82 125.88) (end 106.66 125.88) (width 0.2) (layer "F.Cu") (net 11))
 (segment (start 134 105.7) (end 113.82 125.88) (width 0.2) (layer "F.Cu") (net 11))
 (segment (start 86.96 101.42) (end 91.363 97.017) (width 0.2) (layer "F.Cu") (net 3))
 (segment (start 136.352 106.501626) (end 134.613626 108.24) (width 0.2) (layer "F.Cu") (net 3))
 (segment (start 136.352 99.818374) (end 136.352 106.501626) (width 0.2) (layer "F.Cu") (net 3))
 (segment (start 133.55969 99.557) (end 136.090626 99.557) (width 0.2) (layer "F.Cu") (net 3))
 (segment (start 131.01969 97.017) (end 133.55969 99.557) (width 0.2) (layer "F.Cu") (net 3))
 (segment (start 134.613626 108.24) (end 134 108.24) (width 0.2) (layer "F.Cu") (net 3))
 (segment (start 91.363 97.017) (end 131.01969 97.017) (width 0.2) (layer "F.Cu") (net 3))
 (segment (start 136.090626 99.557) (end 136.352 99.818374) (width 0.2) (layer "F.Cu") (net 3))
 (segment (start 105.96 101.42) (end 112.78 108.24) (width 0.2) (layer "F.Cu") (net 10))
 (segment (start 112.78 108.24) (end 118.76 108.24) (width 0.2) (layer "F.Cu") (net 10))
 (segment (start 118.76 95.54) (end 79.378 95.54) (width 0.2) (layer "F.Cu") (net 7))
 (segment (start 65.398 109.52) (end 58 109.52) (width 0.2) (layer "F.Cu") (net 7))
 (segment (start 79.378 95.54) (end 65.398 109.52) (width 0.2) (layer "F.Cu") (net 7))
 (segment (start 118.76 93) (end 69.52 93) (width 0.2) (layer "F.Cu") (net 6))
 (segment (start 69.52 93) (end 58 104.52) (width 0.2) (layer "F.Cu") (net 6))
 (segment (start 117.697 99.143) (end 118.76 98.08) (width 0.2) (layer "B.Cu") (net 4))
 (segment (start 118.04 128.92) (end 117.697 128.577) (width 0.2) (layer "B.Cu") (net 4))
 (segment (start 117.697 128.577) (end 117.697 99.143) (width 0.2) (layer "B.Cu") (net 4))
 (segment (start 86.139 126.500314) (end 86.139 120.420314) (width 0.2) (layer "F.Cu") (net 5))
 (segment (start 86.959686 127.321) (end 86.139 126.500314) (width 0.2) (layer "F.Cu") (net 5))
 (segment (start 104.559 102.000314) (end 104.559 100.839686) (width 0.2) (layer "F.Cu") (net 5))
 (segment (start 118.04 133.92) (end 94.719314 133.92) (width 0.2) (layer "F.Cu") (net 5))
 (segment (start 104.559 100.839686) (end 105.379686 100.019) (width 0.2) (layer "F.Cu") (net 5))
 (segment (start 105.379686 100.019) (end 118.159 100.019) (width 0.2) (layer "F.Cu") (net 5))
 (segment (start 94.719314 133.92) (end 88.120314 127.321) (width 0.2) (layer "F.Cu") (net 5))
 (segment (start 88.120314 127.321) (end 86.959686 127.321) (width 0.2) (layer "F.Cu") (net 5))
 (segment (start 118.159 100.019) (end 118.76 100.62) (width 0.2) (layer "F.Cu") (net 5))
 (segment (start 86.139 120.420314) (end 104.559 102.000314) (width 0.2) (layer "F.Cu") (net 5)))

